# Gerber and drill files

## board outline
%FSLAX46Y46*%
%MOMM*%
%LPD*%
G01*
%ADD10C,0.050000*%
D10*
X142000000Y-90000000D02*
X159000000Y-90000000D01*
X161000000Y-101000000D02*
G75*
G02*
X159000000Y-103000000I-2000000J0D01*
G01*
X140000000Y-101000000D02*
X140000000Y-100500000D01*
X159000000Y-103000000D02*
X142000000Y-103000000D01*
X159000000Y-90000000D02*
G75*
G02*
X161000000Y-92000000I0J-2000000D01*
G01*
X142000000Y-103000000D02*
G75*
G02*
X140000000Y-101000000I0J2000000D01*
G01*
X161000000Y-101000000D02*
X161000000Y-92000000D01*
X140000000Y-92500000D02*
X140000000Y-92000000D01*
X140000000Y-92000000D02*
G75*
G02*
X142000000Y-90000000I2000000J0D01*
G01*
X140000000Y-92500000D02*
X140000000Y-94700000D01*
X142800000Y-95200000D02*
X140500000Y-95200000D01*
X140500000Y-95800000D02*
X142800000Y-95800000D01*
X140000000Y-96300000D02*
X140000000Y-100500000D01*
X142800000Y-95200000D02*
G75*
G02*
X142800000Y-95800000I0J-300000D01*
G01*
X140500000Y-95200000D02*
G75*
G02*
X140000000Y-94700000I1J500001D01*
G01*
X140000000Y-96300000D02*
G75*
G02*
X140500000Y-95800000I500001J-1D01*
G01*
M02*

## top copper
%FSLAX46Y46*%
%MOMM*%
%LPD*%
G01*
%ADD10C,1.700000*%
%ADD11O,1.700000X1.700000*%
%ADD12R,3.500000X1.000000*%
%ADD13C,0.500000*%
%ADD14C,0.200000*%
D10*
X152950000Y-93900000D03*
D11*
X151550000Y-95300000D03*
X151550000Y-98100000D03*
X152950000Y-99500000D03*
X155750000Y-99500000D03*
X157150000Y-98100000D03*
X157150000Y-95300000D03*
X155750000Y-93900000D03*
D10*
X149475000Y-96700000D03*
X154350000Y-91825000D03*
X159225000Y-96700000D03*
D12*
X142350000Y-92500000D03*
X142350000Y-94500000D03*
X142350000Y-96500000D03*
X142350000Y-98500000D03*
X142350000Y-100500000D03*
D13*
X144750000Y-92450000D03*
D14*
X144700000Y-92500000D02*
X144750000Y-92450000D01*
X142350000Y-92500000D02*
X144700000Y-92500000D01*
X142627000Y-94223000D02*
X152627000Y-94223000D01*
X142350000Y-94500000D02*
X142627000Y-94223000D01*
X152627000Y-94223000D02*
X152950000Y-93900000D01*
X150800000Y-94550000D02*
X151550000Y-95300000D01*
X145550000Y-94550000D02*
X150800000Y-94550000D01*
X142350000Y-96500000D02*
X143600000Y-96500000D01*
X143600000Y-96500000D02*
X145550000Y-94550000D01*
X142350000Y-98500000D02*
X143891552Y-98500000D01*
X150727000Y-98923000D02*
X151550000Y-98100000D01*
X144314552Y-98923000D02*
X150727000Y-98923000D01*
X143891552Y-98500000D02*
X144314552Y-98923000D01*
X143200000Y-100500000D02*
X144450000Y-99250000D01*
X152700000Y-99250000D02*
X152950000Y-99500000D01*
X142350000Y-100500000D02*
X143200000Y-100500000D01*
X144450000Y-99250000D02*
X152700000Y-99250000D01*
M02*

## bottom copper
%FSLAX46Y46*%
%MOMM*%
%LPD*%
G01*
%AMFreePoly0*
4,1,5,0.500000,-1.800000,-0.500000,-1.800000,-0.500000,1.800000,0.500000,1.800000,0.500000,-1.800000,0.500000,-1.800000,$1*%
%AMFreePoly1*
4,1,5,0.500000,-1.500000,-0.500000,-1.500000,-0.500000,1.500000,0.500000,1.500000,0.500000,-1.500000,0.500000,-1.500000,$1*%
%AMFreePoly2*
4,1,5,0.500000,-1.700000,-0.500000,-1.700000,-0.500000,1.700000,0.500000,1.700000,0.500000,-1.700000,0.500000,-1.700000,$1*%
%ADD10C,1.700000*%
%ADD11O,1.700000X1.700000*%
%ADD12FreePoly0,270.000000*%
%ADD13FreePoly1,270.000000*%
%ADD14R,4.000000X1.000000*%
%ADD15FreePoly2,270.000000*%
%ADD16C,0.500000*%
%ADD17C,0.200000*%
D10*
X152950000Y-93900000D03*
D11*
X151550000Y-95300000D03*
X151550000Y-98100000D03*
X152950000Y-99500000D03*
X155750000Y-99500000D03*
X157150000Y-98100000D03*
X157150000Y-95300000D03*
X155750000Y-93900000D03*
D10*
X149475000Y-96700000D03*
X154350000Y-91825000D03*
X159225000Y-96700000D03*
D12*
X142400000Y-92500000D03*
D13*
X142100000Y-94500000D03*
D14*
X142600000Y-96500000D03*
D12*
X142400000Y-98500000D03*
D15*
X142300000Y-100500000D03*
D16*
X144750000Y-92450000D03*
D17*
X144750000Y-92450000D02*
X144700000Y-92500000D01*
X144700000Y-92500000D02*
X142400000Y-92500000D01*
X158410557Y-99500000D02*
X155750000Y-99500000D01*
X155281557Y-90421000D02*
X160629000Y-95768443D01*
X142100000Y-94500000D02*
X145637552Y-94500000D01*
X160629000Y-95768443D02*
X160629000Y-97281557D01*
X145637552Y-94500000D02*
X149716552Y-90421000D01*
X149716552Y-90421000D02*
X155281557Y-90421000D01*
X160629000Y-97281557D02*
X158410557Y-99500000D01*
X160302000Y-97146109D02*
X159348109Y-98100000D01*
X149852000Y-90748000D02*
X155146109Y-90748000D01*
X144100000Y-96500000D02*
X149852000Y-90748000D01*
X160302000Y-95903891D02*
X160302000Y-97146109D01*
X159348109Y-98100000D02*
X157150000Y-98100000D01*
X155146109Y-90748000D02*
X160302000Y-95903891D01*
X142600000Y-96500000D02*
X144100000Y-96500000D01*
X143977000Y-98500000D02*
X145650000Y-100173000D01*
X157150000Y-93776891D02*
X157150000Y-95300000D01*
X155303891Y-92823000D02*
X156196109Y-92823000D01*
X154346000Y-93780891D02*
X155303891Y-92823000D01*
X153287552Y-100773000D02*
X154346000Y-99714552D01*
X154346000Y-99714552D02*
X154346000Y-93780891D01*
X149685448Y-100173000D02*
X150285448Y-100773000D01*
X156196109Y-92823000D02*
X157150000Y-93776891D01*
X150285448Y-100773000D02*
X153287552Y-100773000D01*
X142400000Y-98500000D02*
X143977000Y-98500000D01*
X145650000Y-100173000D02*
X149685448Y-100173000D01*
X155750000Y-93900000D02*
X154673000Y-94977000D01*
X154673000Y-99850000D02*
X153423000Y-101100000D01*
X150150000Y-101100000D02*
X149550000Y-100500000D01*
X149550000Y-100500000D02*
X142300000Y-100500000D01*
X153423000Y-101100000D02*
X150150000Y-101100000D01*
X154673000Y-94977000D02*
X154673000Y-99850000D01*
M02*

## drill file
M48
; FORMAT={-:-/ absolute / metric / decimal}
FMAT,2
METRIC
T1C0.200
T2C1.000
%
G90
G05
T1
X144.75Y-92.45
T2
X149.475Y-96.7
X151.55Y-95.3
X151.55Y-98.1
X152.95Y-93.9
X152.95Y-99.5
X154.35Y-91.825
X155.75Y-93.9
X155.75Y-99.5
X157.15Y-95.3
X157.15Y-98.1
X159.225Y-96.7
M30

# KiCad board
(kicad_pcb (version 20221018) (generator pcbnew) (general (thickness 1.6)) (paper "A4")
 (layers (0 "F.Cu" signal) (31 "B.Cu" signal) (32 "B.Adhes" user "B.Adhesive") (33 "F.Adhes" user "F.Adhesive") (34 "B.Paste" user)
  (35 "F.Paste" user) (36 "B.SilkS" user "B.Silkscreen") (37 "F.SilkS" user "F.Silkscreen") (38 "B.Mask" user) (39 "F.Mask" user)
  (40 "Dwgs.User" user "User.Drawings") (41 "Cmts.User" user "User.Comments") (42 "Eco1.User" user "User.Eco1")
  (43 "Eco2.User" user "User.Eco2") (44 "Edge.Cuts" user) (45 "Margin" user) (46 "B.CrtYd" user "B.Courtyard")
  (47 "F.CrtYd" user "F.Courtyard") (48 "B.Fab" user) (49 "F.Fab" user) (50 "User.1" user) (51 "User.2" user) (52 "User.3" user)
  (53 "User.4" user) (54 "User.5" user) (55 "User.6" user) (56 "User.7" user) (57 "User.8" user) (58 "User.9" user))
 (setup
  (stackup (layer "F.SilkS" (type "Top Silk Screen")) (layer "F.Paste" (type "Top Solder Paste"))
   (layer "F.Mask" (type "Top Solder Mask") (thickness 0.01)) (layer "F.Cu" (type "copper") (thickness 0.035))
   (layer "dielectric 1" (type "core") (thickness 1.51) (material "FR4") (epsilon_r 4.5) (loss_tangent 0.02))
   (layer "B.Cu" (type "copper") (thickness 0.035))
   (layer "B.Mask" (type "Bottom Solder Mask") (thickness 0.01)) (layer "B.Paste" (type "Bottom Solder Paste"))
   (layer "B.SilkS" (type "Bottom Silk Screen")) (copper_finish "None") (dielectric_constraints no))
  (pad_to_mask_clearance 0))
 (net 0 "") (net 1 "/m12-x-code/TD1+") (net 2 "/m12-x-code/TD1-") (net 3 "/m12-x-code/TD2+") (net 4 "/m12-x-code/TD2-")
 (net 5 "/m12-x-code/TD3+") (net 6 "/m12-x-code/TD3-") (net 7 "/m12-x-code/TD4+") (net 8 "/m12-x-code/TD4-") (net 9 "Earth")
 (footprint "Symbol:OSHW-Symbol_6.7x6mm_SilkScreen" (layer "F.Cu") (at 147.75 99.95)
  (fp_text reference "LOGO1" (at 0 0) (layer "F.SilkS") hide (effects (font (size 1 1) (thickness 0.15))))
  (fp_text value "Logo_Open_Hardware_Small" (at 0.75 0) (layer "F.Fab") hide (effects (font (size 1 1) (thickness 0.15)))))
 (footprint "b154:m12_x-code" (layer "F.Cu") (at 154.35 96.7)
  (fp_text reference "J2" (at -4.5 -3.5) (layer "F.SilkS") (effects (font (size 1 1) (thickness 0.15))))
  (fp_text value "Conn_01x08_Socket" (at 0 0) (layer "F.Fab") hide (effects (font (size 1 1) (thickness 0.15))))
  (pad "1" thru_hole circle (at -1.4 -2.8) (size 1.7 1.7) (drill 1) (layers "*.Cu" "*.Mask") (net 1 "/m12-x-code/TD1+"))
  (pad "2" thru_hole oval (at -2.8 -1.4) (size 1.7 1.7) (drill 1) (layers "*.Cu" "*.Mask") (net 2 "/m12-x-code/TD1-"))
  (pad "3" thru_hole oval (at -2.8 1.4) (size 1.7 1.7) (drill 1) (layers "*.Cu" "*.Mask") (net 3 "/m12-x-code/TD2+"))
  (pad "4" thru_hole oval (at -1.4 2.8) (size 1.7 1.7) (drill 1) (layers "*.Cu" "*.Mask") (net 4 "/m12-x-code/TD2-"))
  (pad "5" thru_hole oval (at 1.4 2.8) (size 1.7 1.7) (drill 1) (layers "*.Cu" "*.Mask") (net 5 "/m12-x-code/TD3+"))
  (pad "6" thru_hole oval (at 2.8 1.4) (size 1.7 1.7) (drill 1) (layers "*.Cu" "*.Mask") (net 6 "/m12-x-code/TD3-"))
  (pad "7" thru_hole oval (at 2.8 -1.4) (size 1.7 1.7) (drill 1) (layers "*.Cu" "*.Mask") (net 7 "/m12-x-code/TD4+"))
  (pad "8" thru_hole oval (at 1.4 -2.8) (size 1.7 1.7) (drill 1) (layers "*.Cu" "*.Mask") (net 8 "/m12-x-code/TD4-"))
  (pad "S" thru_hole circle (at -4.875 0) (size 1.7 1.7) (drill 1) (layers "*.Cu" "*.Mask"))
  (pad "S" thru_hole circle (at 0 -4.875) (size 1.7 1.7) (drill 1) (layers "*.Cu" "*.Mask"))
  (pad "S" thru_hole circle (at 4.875 0) (size 1.7 1.7) (drill 1) (layers "*.Cu" "*.Mask")))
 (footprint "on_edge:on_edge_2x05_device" (layer "F.Cu") (at 140 96.5 -90)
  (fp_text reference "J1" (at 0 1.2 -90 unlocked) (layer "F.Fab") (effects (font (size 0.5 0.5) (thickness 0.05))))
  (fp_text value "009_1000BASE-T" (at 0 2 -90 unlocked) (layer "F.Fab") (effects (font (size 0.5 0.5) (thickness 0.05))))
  (fp_line (start -4 0) (end -1.8 0) (stroke (width 0.05) (type solid)) (layer "Edge.Cuts"))
  (fp_line (start -1.3 -2.8) (end -1.3 -0.5) (stroke (width 0.05) (type solid)) (layer "Edge.Cuts"))
  (fp_line (start -0.7 -0.5) (end -0.7 -2.8) (stroke (width 0.05) (type solid)) (layer "Edge.Cuts"))
  (fp_line (start -0.2 0) (end 4 0) (stroke (width 0.05) (type solid)) (layer "Edge.Cuts"))
  (fp_arc (start -1.3 -2.8) (mid -1 -3.1) (end -0.7 -2.8) (stroke (width 0.05) (type solid)) (layer "Edge.Cuts"))
  (fp_arc (start -1.3 -0.5) (mid -1.446447 -0.146447) (end -1.8 0) (stroke (width 0.05) (type solid)) (layer "Edge.Cuts"))
  (fp_arc (start -0.2 0) (mid -0.553553 -0.146447) (end -0.7 -0.5) (stroke (width 0.05) (type solid)) (layer "Edge.Cuts"))
  (pad "1" smd rect (at -4 -2.35 90) (size 1 3.5) (layers "F.Cu" "F.Mask") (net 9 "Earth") (zone_connect 0))
  (pad "2" smd rect (at -2 -2.35 270) (size 1 3.5) (layers "F.Cu" "F.Mask") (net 1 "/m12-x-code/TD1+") (zone_connect 0))
  (pad "3" smd rect (at 0 -2.35 270) (size 1 3.5) (layers "F.Cu" "F.Mask") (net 2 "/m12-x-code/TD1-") (zone_connect 0))
  (pad "4" smd rect (at 2 -2.35 90) (size 1 3.5) (layers "F.Cu" "F.Mask") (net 3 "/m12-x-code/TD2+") (zone_connect 0))
  (pad "5" smd rect (at 4 -2.35 90) (size 1 3.5) (layers "F.Cu" "F.Mask") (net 4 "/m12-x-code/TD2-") (zone_connect 0))
  (pad "6" smd custom (at -4 -2.4 270) (size 1 3.6) (layers "B.Cu" "B.Mask") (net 9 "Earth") (zone_connect 0)
   (options (clearance outline) (anchor rect)) (primitives))
  (pad "7" smd custom (at -2 -2.1 270) (size 1 3) (layers "B.Cu" "B.Mask") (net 5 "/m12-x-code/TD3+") (zone_connect 0)
   (options (clearance outline) (anchor rect)) (primitives))
  (pad "8" smd rect (at 0 -2.6 270) (size 1 4) (layers "B.Cu" "B.Mask") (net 6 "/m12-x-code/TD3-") (zone_connect 0))
  (pad "9" smd custom (at 2 -2.4 270) (size 1 3.6) (layers "B.Cu" "B.Mask") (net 7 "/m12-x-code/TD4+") (zone_connect 0)
   (options (clearance outline) (anchor rect)) (primitives))
  (pad "10" smd custom (at 4 -2.3 270) (size 1 3.4) (layers "B.Cu" "B.Mask") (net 8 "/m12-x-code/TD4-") (zone_connect 0)
   (options (clearance outline) (anchor rect)) (primitives))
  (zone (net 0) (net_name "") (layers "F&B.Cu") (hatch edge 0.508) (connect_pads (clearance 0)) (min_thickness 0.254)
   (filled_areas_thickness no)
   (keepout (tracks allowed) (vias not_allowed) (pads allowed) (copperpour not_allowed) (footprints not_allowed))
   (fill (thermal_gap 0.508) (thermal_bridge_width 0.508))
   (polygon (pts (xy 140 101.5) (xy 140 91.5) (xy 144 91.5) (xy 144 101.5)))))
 (gr_line (start 142 90) (end 159 90) (stroke (width 0.05) (type solid)) (layer "Edge.Cuts"))
 (gr_arc (start 161 101) (mid 160.414214 102.414214) (end 159 103) (stroke (width 0.05) (type solid)) (layer "Edge.Cuts"))
 (gr_line (start 140 101) (end 140 100.5) (stroke (width 0.05) (type solid)) (layer "Edge.Cuts"))
 (gr_line (start 159 103) (end 142 103) (stroke (width 0.05) (type solid)) (layer "Edge.Cuts"))
 (gr_arc (start 159 90) (mid 160.414214 90.585786) (end 161 92) (stroke (width 0.05) (type solid)) (layer "Edge.Cuts"))
 (gr_arc (start 142 103) (mid 140.585786 102.414214) (end 140 101) (stroke (width 0.05) (type solid)) (layer "Edge.Cuts"))
 (gr_line (start 161 101) (end 161 92) (stroke (width 0.05) (type solid)) (layer "Edge.Cuts"))
 (gr_line (start 140 92.5) (end 140 92) (stroke (width 0.05) (type solid)) (layer "Edge.Cuts"))
 (gr_arc (start 140 92) (mid 140.585786 90.585786) (end 142 90) (stroke (width 0.05) (type solid)) (layer "Edge.Cuts"))
 (segment (start 144.7 92.5) (end 144.75 92.45) (width 0.2) (layer "F.Cu") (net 9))
 (segment (start 142.35 92.5) (end 144.7 92.5) (width 0.2) (layer "F.Cu") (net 9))
 (via (at 144.75 92.45) (size 0.5) (drill 0.2) (layers "F.Cu" "B.Cu") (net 9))
 (segment (start 144.75 92.45) (end 144.7 92.5) (width 0.2) (layer "B.Cu") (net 9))
 (segment (start 144.7 92.5) (end 142.4 92.5) (width 0.2) (layer "B.Cu") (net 9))
 (segment (start 142.627 94.223) (end 152.627 94.223) (width 0.2) (layer "F.Cu") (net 1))
 (segment (start 142.35 94.5) (end 142.627 94.223) (width 0.2) (layer "F.Cu") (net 1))
 (segment (start 152.627 94.223) (end 152.95 93.9) (width 0.2) (layer "F.Cu") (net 1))
 (segment (start 150.8 94.55) (end 151.55 95.3) (width 0.2) (layer "F.Cu") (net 2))
 (segment (start 145.55 94.55) (end 150.8 94.55) (width 0.2) (layer "F.Cu") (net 2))
 (segment (start 142.35 96.5) (end 143.6 96.5) (width 0.2) (layer "F.Cu") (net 2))
 (segment (start 143.6 96.5) (end 145.55 94.55) (width 0.2) (layer "F.Cu") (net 2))
 (segment (start 142.35 98.5) (end 143.891552 98.5) (width 0.2) (layer "F.Cu") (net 3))
 (segment (start 150.727 98.923) (end 151.55 98.1) (width 0.2) (layer "F.Cu") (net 3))
 (segment (start 144.314552 98.923) (end 150.727 98.923) (width 0.2) (layer "F.Cu") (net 3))
 (segment (start 143.891552 98.5) (end 144.314552 98.923) (width 0.2) (layer "F.Cu") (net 3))
 (segment (start 143.2 100.5) (end 144.45 99.25) (width 0.2) (layer "F.Cu") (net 4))
 (segment (start 152.7 99.25) (end 152.95 99.5) (width 0.2) (layer "F.Cu") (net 4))
 (segment (start 142.35 100.5) (end 143.2 100.5) (width 0.2) (layer "F.Cu") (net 4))
 (segment (start 144.45 99.25) (end 152.7 99.25) (width 0.2) (layer "F.Cu") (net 4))
 (segment (start 158.410557 99.5) (end 155.75 99.5) (width 0.2) (layer "B.Cu") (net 5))
 (segment (start 155.281557 90.421) (end 160.629 95.768443) (width 0.2) (layer "B.Cu") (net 5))
 (segment (start 142.1 94.5) (end 145.637552 94.5) (width 0.2) (layer "B.Cu") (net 5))
 (segment (start 160.629 95.768443) (end 160.629 97.281557) (width 0.2) (layer "B.Cu") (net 5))
 (segment (start 145.637552 94.5) (end 149.716552 90.421) (width 0.2) (layer "B.Cu") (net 5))
 (segment (start 149.716552 90.421) (end 155.281557 90.421) (width 0.2) (layer "B.Cu") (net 5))
 (segment (start 160.629 97.281557) (end 158.410557 99.5) (width 0.2) (layer "B.Cu") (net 5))
 (segment (start 160.302 97.146109) (end 159.348109 98.1) (width 0.2) (layer "B.Cu") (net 6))
 (segment (start 149.852 90.748) (end 155.146109 90.748) (width 0.2) (layer "B.Cu") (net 6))
 (segment (start 144.1 96.5) (end 149.852 90.748) (width 0.2) (layer "B.Cu") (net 6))
 (segment (start 160.302 95.903891) (end 160.302 97.146109) (width 0.2) (layer "B.Cu") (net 6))
 (segment (start 159.348109 98.1) (end 157.15 98.1) (width 0.2) (layer "B.Cu") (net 6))
 (segment (start 155.146109 90.748) (end 160.302 95.903891) (width 0.2) (layer "B.Cu") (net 6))
 (segment (start 142.6 96.5) (end 144.1 96.5) (width 0.2) (layer "B.Cu") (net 6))
 (segment (start 143.977 98.5) (end 145.65 100.173) (width 0.2) (layer "B.Cu") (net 7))
 (segment (start 157.15 93.776891) (end 157.15 95.3) (width 0.2) (layer "B.Cu") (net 7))
 (segment (start 155.303891 92.823) (end 156.196109 92.823) (width 0.2) (layer "B.Cu") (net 7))
 (segment (start 154.346 93.780891) (end 155.303891 92.823) (width 0.2) (layer "B.Cu") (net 7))
 (segment (start 153.287552 100.773) (end 154.346 99.714552) (width 0.2) (layer "B.Cu") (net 7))
 (segment (start 154.346 99.714552) (end 154.346 93.780891) (width 0.2) (layer "B.Cu") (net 7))
 (segment (start 149.685448 100.173) (end 150.285448 100.773) (width 0.2) (layer "B.Cu") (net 7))
 (segment (start 156.196109 92.823) (end 157.15 93.776891) (width 0.2) (layer "B.Cu") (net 7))
 (segment (start 150.285448 100.773) (end 153.287552 100.773) (width 0.2) (layer "B.Cu") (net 7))
 (segment (start 142.4 98.5) (end 143.977 98.5) (width 0.2) (layer "B.Cu") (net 7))
 (segment (start 145.65 100.173) (end 149.685448 100.173) (width 0.2) (layer "B.Cu") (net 7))
 (segment (start 155.75 93.9) (end 154.673 94.977) (width 0.2) (layer "B.Cu") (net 8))
 (segment (start 154.673 99.85) (end 153.423 101.1) (width 0.2) (layer "B.Cu") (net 8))
 (segment (start 150.15 101.1) (end 149.55 100.5) (width 0.2) (layer "B.Cu") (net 8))
 (segment (start 149.55 100.5) (end 142.3 100.5) (width 0.2) (layer "B.Cu") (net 8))
 (segment (start 153.423 101.1) (end 150.15 101.1) (width 0.2) (layer "B.Cu") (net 8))
 (segment (start 154.673 94.977) (end 154.673 99.85) (width 0.2) (layer "B.Cu") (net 8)))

